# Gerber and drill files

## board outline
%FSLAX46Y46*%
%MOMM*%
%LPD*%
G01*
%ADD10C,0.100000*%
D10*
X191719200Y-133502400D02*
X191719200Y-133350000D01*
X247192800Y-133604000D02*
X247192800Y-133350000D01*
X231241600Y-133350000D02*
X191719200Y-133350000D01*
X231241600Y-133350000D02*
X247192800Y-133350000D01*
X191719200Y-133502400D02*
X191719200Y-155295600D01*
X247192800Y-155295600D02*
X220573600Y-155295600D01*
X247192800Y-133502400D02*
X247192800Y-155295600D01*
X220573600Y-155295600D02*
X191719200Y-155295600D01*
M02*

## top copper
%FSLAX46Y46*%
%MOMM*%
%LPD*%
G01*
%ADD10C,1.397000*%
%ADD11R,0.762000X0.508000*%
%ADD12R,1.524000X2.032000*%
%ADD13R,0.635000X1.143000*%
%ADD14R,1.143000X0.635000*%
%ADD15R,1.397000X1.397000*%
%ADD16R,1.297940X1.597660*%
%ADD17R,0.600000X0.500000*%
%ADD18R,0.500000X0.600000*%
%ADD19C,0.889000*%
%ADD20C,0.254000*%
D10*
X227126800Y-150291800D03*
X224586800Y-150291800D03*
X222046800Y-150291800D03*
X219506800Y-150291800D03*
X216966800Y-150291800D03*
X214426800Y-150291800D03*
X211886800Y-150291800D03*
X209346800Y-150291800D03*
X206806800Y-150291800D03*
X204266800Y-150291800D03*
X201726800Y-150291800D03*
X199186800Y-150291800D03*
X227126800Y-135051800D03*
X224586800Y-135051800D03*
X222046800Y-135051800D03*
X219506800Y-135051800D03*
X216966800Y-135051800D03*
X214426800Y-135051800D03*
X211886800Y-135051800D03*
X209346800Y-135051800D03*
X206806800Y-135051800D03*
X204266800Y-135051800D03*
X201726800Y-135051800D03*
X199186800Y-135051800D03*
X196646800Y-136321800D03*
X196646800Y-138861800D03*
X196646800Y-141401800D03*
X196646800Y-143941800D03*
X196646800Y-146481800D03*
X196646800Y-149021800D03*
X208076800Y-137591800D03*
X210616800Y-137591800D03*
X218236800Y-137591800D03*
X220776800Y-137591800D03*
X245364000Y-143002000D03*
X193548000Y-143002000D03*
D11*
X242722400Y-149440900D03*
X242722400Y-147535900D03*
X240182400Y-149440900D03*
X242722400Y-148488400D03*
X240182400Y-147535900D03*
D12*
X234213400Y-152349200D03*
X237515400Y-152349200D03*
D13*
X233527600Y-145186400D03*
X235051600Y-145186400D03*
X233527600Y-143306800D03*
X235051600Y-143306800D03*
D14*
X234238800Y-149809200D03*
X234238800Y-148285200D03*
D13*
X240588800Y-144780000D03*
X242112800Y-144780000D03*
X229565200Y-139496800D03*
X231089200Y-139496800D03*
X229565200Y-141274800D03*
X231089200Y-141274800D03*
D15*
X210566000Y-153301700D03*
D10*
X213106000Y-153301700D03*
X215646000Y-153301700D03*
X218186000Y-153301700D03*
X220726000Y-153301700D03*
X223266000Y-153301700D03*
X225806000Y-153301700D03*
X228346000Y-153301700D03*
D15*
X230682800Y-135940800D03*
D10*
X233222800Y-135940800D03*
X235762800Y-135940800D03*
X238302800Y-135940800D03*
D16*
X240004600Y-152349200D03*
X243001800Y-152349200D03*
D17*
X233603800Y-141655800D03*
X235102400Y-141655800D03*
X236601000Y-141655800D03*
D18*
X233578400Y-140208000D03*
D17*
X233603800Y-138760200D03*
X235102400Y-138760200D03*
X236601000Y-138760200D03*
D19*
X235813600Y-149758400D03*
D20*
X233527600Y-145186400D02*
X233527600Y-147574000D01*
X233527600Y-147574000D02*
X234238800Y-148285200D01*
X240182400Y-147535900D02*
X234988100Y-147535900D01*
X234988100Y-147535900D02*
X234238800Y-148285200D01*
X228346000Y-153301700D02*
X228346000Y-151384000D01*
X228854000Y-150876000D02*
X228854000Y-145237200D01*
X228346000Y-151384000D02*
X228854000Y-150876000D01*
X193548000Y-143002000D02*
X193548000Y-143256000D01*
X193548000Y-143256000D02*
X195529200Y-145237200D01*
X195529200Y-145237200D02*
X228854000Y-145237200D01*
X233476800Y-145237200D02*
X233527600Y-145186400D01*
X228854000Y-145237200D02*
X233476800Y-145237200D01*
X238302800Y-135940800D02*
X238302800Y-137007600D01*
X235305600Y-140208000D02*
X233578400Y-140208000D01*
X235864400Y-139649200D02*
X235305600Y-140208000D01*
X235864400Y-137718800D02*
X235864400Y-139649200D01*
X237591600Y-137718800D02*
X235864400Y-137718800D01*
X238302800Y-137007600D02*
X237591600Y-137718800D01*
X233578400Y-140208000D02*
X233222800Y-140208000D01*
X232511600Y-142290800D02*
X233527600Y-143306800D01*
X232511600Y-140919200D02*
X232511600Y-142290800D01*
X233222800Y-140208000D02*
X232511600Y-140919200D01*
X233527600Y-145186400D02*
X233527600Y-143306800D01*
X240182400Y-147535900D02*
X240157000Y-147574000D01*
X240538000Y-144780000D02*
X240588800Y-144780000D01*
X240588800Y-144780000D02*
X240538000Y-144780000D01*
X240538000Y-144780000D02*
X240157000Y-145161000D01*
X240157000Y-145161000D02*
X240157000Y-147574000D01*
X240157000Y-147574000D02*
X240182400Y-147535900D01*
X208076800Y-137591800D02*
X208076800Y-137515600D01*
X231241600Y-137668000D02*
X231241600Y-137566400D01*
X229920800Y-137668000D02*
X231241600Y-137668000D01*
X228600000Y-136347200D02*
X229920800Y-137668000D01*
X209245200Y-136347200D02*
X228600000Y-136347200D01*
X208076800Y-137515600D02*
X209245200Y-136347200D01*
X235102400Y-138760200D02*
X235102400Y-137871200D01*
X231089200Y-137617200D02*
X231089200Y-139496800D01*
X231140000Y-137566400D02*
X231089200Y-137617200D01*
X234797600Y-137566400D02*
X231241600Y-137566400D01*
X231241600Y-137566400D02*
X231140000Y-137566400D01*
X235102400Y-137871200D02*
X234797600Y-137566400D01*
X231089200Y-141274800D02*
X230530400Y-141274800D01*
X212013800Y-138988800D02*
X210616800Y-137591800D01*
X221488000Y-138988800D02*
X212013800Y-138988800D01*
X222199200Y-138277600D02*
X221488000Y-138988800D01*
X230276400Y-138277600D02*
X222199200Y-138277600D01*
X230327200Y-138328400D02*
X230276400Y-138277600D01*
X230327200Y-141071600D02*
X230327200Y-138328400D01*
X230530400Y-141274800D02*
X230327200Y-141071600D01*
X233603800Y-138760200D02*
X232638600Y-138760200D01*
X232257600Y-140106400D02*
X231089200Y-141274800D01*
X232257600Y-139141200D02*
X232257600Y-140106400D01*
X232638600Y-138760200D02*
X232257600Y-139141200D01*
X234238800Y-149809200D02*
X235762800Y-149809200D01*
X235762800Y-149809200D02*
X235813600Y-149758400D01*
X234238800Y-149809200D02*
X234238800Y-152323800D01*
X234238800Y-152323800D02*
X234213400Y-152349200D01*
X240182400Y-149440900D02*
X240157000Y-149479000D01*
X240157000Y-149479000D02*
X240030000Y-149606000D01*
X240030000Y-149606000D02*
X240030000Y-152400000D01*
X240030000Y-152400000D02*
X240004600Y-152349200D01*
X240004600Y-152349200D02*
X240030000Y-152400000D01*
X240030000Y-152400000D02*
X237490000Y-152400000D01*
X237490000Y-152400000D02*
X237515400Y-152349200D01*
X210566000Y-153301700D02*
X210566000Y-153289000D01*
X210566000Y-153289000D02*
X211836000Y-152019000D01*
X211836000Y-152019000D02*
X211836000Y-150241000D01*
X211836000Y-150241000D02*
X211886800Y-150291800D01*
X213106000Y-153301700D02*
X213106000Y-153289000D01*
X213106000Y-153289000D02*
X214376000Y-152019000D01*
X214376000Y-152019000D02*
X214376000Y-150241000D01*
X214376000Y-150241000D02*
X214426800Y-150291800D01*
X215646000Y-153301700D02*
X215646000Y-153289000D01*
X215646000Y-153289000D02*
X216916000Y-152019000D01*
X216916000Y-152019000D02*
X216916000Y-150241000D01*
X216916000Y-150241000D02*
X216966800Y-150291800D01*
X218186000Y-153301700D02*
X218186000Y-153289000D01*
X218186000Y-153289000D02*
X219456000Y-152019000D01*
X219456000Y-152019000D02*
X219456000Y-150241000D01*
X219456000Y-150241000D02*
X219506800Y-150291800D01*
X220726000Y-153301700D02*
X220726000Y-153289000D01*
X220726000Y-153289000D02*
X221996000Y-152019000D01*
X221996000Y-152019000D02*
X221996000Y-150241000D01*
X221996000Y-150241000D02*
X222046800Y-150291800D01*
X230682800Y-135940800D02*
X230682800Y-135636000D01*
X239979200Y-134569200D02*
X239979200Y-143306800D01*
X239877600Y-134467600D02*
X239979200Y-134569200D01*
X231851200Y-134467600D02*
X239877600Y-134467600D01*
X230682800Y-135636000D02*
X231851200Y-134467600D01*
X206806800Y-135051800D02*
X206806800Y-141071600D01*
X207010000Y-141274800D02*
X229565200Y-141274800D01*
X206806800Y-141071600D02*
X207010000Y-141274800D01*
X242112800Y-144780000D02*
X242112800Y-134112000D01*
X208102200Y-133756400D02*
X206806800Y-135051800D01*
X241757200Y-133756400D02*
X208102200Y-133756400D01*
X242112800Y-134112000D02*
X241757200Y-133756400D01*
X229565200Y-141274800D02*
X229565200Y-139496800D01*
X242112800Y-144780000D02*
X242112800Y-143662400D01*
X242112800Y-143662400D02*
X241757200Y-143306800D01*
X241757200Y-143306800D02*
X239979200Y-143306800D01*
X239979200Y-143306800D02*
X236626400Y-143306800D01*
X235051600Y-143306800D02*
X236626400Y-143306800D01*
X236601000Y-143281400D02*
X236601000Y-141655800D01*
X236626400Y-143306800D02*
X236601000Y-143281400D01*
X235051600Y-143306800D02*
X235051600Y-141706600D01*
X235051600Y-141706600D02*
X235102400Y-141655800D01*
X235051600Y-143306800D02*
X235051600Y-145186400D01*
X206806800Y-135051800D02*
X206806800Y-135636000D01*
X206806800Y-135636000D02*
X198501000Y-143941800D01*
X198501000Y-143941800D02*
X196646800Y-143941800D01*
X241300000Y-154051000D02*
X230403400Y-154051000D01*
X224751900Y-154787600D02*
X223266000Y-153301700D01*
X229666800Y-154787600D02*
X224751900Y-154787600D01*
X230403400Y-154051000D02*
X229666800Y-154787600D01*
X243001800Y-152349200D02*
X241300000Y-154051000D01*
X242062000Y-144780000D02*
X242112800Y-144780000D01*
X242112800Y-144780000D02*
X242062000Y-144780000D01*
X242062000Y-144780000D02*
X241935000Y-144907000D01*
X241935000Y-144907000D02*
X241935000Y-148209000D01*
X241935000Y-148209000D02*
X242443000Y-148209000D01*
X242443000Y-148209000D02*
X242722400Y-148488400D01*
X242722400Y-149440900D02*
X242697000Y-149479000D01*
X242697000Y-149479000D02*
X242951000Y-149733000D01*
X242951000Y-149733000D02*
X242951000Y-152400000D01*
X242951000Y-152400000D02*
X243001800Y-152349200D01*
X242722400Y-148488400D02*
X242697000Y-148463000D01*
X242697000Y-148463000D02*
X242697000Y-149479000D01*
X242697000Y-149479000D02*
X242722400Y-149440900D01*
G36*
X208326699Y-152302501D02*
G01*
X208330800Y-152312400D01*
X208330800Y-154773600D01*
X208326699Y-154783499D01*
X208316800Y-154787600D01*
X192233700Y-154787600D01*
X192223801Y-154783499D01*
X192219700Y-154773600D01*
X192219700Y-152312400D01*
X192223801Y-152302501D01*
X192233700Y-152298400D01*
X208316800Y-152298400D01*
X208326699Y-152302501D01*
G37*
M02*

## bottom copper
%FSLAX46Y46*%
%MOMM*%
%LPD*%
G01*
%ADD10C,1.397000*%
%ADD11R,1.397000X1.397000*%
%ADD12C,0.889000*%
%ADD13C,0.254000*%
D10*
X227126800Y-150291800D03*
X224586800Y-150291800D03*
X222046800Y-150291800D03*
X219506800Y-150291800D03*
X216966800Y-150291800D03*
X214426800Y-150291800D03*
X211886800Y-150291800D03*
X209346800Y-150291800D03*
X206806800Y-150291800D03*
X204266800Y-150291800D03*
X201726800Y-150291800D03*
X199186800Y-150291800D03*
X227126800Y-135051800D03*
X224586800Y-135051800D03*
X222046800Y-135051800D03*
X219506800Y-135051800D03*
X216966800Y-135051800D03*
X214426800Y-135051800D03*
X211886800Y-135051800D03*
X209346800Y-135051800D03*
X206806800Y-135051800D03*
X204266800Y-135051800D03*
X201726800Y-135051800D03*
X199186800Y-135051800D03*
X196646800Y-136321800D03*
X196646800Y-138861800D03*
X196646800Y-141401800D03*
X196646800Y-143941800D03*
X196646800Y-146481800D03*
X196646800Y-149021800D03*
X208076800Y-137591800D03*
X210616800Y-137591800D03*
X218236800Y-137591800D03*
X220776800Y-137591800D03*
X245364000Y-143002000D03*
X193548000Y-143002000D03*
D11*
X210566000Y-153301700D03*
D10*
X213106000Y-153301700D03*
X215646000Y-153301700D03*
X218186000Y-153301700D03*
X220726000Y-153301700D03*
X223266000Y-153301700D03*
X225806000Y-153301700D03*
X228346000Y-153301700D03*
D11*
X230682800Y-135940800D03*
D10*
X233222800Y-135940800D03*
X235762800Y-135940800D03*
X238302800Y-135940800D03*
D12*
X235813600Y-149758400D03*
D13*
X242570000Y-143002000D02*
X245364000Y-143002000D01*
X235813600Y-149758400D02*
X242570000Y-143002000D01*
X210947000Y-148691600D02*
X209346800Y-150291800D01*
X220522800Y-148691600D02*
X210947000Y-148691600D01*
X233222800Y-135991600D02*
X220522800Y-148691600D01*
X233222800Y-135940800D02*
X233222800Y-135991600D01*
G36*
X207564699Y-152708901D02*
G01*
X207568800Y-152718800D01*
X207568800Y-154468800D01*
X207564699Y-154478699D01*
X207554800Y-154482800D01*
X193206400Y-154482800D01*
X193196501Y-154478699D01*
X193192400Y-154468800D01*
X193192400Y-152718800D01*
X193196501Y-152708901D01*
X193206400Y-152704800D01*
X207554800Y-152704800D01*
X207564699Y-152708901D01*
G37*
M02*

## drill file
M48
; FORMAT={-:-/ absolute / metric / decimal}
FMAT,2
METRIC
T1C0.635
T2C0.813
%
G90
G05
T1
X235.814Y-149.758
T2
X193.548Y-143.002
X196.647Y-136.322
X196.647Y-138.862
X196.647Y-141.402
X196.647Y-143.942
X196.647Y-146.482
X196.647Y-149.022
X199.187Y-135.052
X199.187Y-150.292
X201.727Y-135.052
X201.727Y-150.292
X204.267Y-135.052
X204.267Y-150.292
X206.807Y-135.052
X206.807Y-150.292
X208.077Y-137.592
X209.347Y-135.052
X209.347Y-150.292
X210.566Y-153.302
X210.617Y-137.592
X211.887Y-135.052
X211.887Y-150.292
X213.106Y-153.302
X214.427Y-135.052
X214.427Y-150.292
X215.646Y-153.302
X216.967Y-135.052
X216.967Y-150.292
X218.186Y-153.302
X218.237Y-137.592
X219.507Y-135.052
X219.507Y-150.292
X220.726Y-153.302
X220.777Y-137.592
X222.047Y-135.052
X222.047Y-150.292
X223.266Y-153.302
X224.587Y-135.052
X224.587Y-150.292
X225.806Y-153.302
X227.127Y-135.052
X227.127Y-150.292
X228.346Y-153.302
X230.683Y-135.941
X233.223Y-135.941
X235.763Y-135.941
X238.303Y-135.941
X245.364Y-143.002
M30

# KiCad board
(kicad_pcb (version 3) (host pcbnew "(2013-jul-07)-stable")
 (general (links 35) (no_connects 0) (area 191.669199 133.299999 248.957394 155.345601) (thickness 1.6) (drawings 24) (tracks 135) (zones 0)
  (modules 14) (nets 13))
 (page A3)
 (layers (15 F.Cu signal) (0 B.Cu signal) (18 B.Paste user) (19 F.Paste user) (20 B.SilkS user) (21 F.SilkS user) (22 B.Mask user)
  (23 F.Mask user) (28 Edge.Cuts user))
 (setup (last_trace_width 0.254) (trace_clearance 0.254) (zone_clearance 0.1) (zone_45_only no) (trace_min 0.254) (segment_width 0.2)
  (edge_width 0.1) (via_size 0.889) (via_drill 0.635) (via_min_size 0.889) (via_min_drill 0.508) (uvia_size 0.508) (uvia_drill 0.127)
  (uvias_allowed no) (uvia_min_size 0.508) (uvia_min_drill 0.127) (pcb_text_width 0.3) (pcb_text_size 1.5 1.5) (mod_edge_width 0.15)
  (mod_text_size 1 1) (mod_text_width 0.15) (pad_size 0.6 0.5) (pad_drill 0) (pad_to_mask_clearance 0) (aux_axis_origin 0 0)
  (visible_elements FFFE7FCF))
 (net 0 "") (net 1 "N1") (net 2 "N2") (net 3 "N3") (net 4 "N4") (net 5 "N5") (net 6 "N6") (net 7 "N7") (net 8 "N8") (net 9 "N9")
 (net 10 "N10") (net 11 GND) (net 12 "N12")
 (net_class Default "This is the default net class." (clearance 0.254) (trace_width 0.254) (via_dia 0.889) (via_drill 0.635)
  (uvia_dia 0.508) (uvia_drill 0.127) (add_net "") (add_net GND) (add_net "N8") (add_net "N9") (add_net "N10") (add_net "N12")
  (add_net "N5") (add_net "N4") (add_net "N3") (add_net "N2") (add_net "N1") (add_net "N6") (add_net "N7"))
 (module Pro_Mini (layer F.Cu) (at 211.9884 142.6972)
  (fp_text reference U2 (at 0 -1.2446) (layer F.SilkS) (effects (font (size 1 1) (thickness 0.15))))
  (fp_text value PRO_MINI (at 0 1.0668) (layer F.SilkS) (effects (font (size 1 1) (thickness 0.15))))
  (pad 9 thru_hole circle (at 15.1384 7.5946) (size 1.397 1.397) (drill 0.8128) (layers *.Cu *.Mask F.SilkS))
  (pad 8 thru_hole circle (at 12.5984 7.5946) (size 1.397 1.397) (drill 0.8128) (layers *.Cu *.Mask F.SilkS))
  (pad 7 thru_hole circle (at 10.0584 7.5946) (size 1.397 1.397) (drill 0.8128) (layers *.Cu *.Mask F.SilkS) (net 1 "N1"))
  (pad 6 thru_hole circle (at 7.5184 7.5946) (size 1.397 1.397) (drill 0.8128) (layers *.Cu *.Mask F.SilkS) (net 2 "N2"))
  (pad 5 thru_hole circle (at 4.9784 7.5946) (size 1.397 1.397) (drill 0.8128) (layers *.Cu *.Mask F.SilkS) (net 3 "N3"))
  (pad 4 thru_hole circle (at 2.4384 7.5946) (size 1.397 1.397) (drill 0.8128) (layers *.Cu *.Mask F.SilkS) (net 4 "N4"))
  (pad 3 thru_hole circle (at -0.1016 7.5946) (size 1.397 1.397) (drill 0.8128) (layers *.Cu *.Mask F.SilkS) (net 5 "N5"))
  (pad 2 thru_hole circle (at -2.6416 7.5946) (size 1.397 1.397) (drill 0.8128) (layers *.Cu *.Mask F.SilkS) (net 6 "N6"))
  (pad GND thru_hole circle (at -5.1816 7.5946) (size 1.397 1.397) (drill 0.8128) (layers *.Cu *.Mask F.SilkS))
  (pad RST thru_hole circle (at -7.7216 7.5946) (size 1.397 1.397) (drill 0.8128) (layers *.Cu *.Mask F.SilkS))
  (pad RX1 thru_hole circle (at -10.2616 7.5946) (size 1.397 1.397) (drill 0.8128) (layers *.Cu *.Mask F.SilkS))
  (pad TX0 thru_hole circle (at -12.8016 7.5946) (size 1.397 1.397) (drill 0.8128) (layers *.Cu *.Mask F.SilkS))
  (pad 10 thru_hole circle (at 15.1384 -7.6454) (size 1.397 1.397) (drill 0.8128) (layers *.Cu *.Mask F.SilkS))
  (pad 11 thru_hole circle (at 12.5984 -7.6454) (size 1.397 1.397) (drill 0.8128) (layers *.Cu *.Mask F.SilkS))
  (pad 12 thru_hole circle (at 10.0584 -7.6454) (size 1.397 1.397) (drill 0.8128) (layers *.Cu *.Mask F.SilkS))
  (pad 13 thru_hole circle (at 7.5184 -7.6454) (size 1.397 1.397) (drill 0.8128) (layers *.Cu *.Mask F.SilkS))
  (pad A0 thru_hole circle (at 4.9784 -7.6454) (size 1.397 1.397) (drill 0.8128) (layers *.Cu *.Mask F.SilkS))
  (pad A1 thru_hole circle (at 2.4384 -7.6454) (size 1.397 1.397) (drill 0.8128) (layers *.Cu *.Mask F.SilkS))
  (pad A2 thru_hole circle (at -0.1016 -7.6454) (size 1.397 1.397) (drill 0.8128) (layers *.Cu *.Mask F.SilkS))
  (pad A3 thru_hole circle (at -2.6416 -7.6454) (size 1.397 1.397) (drill 0.8128) (layers *.Cu *.Mask F.SilkS))
  (pad VCC thru_hole circle (at -5.1816 -7.6454) (size 1.397 1.397) (drill 0.8128) (layers *.Cu *.Mask F.SilkS) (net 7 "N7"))
  (pad RST thru_hole circle (at -7.7216 -7.6454) (size 1.397 1.397) (drill 0.8128) (layers *.Cu *.Mask F.SilkS))
  (pad GND thru_hole circle (at -10.2616 -7.6454) (size 1.397 1.397) (drill 0.8128) (layers *.Cu *.Mask F.SilkS))
  (pad RAW thru_hole circle (at -12.8016 -7.6454) (size 1.397 1.397) (drill 0.8128) (layers *.Cu *.Mask F.SilkS))
  (pad GRN thru_hole circle (at -15.3416 -6.3754) (size 1.397 1.397) (drill 0.8128) (layers *.Cu *.Mask F.SilkS))
  (pad TX0 thru_hole circle (at -15.3416 -3.8354) (size 1.397 1.397) (drill 0.8128) (layers *.Cu *.Mask F.SilkS))
  (pad RX1 thru_hole circle (at -15.3416 -1.2954) (size 1.397 1.397) (drill 0.8128) (layers *.Cu *.Mask F.SilkS))
  (pad VCC thru_hole circle (at -15.3416 1.2446) (size 1.397 1.397) (drill 0.8128) (layers *.Cu *.Mask F.SilkS) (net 7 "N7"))
  (pad GND thru_hole circle (at -15.3416 3.7846) (size 1.397 1.397) (drill 0.8128) (layers *.Cu *.Mask F.SilkS))
  (pad BLK thru_hole circle (at -15.3416 6.3246) (size 1.397 1.397) (drill 0.8128) (layers *.Cu *.Mask F.SilkS))
  (pad A5 thru_hole circle (at -3.9116 -5.1054) (size 1.397 1.397) (drill 0.8128) (layers *.Cu *.Mask F.SilkS) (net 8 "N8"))
  (pad A4 thru_hole circle (at -1.3716 -5.1054) (size 1.397 1.397) (drill 0.8128) (layers *.Cu *.Mask F.SilkS) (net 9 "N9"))
  (pad A7 thru_hole circle (at 6.2484 -5.1054) (size 1.397 1.397) (drill 0.8128) (layers *.Cu *.Mask F.SilkS))
  (pad A6 thru_hole circle (at 8.7884 -5.1054) (size 1.397 1.397) (drill 0.8128) (layers *.Cu *.Mask F.SilkS)))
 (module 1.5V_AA (layer B.Cu) (at 219.456 143.002)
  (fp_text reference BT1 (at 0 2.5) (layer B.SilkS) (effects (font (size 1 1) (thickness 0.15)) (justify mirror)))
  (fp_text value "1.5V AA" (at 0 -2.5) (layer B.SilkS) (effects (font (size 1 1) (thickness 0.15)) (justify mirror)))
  (pad 1 thru_hole circle (at 25.908 0) (size 1.397 1.397) (drill 0.8128) (layers *.Cu *.Mask B.SilkS) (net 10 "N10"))
  (pad 2 thru_hole circle (at -25.908 0) (size 1.397 1.397) (drill 0.8128) (layers *.Cu *.Mask B.SilkS) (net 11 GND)))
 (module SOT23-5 (layer F.Cu) (at 241.4524 148.4884 90)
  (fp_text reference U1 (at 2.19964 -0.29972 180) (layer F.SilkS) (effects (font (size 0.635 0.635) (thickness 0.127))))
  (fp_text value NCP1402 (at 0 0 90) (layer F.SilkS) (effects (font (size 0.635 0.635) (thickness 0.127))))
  (pad 1 smd rect (at -0.9525 1.27 90) (size 0.508 0.762) (layers F.Cu F.Paste F.Mask) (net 7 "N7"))
  (pad 3 smd rect (at 0.9525 1.27 90) (size 0.508 0.762) (layers F.Cu F.Paste F.Mask))
  (pad 5 smd rect (at -0.9525 -1.27 90) (size 0.508 0.762) (layers F.Cu F.Paste F.Mask) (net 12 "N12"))
  (pad 2 smd rect (at 0 1.27 90) (size 0.508 0.762) (layers F.Cu F.Paste F.Mask) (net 7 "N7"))
  (pad 4 smd rect (at 0.9525 -1.27 90) (size 0.508 0.762) (layers F.Cu F.Paste F.Mask) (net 11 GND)))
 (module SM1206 (layer F.Cu) (at 235.8644 152.3492)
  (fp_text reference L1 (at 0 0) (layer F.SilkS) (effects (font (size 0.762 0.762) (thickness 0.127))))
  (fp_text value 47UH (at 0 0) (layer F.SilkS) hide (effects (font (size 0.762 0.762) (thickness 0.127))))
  (pad 1 smd rect (at -1.651 0) (size 1.524 2.032) (layers F.Cu F.Paste F.Mask) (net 10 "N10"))
  (pad 2 smd rect (at 1.651 0) (size 1.524 2.032) (layers F.Cu F.Paste F.Mask) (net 12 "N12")))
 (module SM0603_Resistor (layer F.Cu) (at 234.2896 145.1864)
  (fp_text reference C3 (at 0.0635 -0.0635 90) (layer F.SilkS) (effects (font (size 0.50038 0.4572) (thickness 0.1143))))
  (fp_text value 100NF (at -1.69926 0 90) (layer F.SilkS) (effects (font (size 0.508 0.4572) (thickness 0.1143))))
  (pad 1 smd rect (at -0.762 0) (size 0.635 1.143) (layers F.Cu F.Paste F.Mask) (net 11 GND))
  (pad 2 smd rect (at 0.762 0) (size 0.635 1.143) (layers F.Cu F.Paste F.Mask) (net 7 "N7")))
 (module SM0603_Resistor (layer F.Cu) (at 234.2896 143.3068)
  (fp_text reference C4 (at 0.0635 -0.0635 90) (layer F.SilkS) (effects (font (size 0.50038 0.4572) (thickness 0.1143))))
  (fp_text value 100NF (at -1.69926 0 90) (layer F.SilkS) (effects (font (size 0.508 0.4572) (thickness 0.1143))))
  (pad 1 smd rect (at -0.762 0) (size 0.635 1.143) (layers F.Cu F.Paste F.Mask) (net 11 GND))
  (pad 2 smd rect (at 0.762 0) (size 0.635 1.143) (layers F.Cu F.Paste F.Mask) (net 7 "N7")))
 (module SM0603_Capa (layer F.Cu) (at 234.2388 149.0472 90)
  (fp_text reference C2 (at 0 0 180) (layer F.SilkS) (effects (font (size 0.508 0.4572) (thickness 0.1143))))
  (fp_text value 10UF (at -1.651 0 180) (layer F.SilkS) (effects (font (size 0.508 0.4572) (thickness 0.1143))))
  (pad 1 smd rect (at -0.762 0 90) (size 0.635 1.143) (layers F.Cu F.Paste F.Mask) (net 10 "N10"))
  (pad 2 smd rect (at 0.762 0 90) (size 0.635 1.143) (layers F.Cu F.Paste F.Mask) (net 11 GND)))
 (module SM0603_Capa (layer F.Cu) (at 241.3508 144.78)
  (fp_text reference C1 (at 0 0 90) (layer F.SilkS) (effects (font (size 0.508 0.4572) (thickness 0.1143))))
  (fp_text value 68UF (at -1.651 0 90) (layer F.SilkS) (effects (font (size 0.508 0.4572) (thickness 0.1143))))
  (pad 1 smd rect (at -0.762 0) (size 0.635 1.143) (layers F.Cu F.Paste F.Mask) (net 11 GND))
  (pad 2 smd rect (at 0.762 0) (size 0.635 1.143) (layers F.Cu F.Paste F.Mask) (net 7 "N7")))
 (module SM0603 (layer F.Cu) (at 230.3272 139.4968)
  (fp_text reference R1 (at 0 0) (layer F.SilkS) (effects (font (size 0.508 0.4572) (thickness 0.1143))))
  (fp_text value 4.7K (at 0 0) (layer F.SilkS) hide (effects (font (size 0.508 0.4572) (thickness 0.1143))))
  (pad 1 smd rect (at -0.762 0) (size 0.635 1.143) (layers F.Cu F.Paste F.Mask) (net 7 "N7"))
  (pad 2 smd rect (at 0.762 0) (size 0.635 1.143) (layers F.Cu F.Paste F.Mask) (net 8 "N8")))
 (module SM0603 (layer F.Cu) (at 230.3272 141.2748)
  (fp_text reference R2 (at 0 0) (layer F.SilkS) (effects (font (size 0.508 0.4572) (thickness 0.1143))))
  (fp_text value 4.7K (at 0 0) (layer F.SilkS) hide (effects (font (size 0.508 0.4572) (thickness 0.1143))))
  (pad 1 smd rect (at -0.762 0) (size 0.635 1.143) (layers F.Cu F.Paste F.Mask) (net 7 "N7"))
  (pad 2 smd rect (at 0.762 0) (size 0.635 1.143) (layers F.Cu F.Paste F.Mask) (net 9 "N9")))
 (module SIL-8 (layer F.Cu) (at 219.456 153.3017)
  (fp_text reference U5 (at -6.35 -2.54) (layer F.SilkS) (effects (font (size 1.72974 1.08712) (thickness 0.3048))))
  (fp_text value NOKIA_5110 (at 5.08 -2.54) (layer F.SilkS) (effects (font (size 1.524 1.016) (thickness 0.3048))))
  (pad 1 thru_hole rect (at -8.89 0) (size 1.397 1.397) (drill 0.8128) (layers *.Cu *.Mask F.SilkS) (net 5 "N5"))
  (pad 2 thru_hole circle (at -6.35 0) (size 1.397 1.397) (drill 0.8128) (layers *.Cu *.Mask F.SilkS) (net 4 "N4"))
  (pad 3 thru_hole circle (at -3.81 0) (size 1.397 1.397) (drill 0.8128) (layers *.Cu *.Mask F.SilkS) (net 3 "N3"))
  (pad 4 thru_hole circle (at -1.27 0) (size 1.397 1.397) (drill 0.8128) (layers *.Cu *.Mask F.SilkS) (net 2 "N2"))
  (pad 5 thru_hole circle (at 1.27 0) (size 1.397 1.397) (drill 0.8128) (layers *.Cu *.Mask F.SilkS) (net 1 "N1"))
  (pad 6 thru_hole circle (at 3.81 0) (size 1.397 1.397) (drill 0.8128) (layers *.Cu *.Mask F.SilkS) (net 7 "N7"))
  (pad 7 thru_hole circle (at 6.35 0) (size 1.397 1.397) (drill 0.8128) (layers *.Cu *.Mask F.SilkS))
  (pad 8 thru_hole circle (at 8.89 0) (size 1.397 1.397) (drill 0.8128) (layers *.Cu *.Mask F.SilkS) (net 11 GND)))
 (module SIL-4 (layer B.Cu) (at 234.4928 135.9408)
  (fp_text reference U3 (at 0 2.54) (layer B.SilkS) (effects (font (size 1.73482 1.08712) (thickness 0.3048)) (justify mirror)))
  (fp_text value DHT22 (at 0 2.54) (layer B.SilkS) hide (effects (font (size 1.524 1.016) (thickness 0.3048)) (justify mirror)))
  (pad 1 thru_hole rect (at -3.81 0) (size 1.397 1.397) (drill 0.8128) (layers *.Cu *.Mask B.SilkS) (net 7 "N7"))
  (pad 2 thru_hole circle (at -1.27 0) (size 1.397 1.397) (drill 0.8128) (layers *.Cu *.Mask B.SilkS) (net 6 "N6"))
  (pad 3 thru_hole circle (at 1.27 0) (size 1.397 1.397) (drill 0.8128) (layers *.Cu *.Mask B.SilkS))
  (pad 4 thru_hole circle (at 3.81 0) (size 1.397 1.397) (drill 0.8128) (layers *.Cu *.Mask B.SilkS) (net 11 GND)))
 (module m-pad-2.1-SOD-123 (layer F.Cu) (at 241.5032 152.3492)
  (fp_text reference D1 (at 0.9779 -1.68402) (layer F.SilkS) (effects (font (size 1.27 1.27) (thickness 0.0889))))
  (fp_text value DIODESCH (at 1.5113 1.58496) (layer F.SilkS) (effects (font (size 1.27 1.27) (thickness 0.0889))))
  (pad 1 smd rect (at -1.4986 0) (size 1.29794 1.59766) (layers F.Cu F.Paste F.Mask) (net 12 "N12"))
  (pad 2 smd rect (at 1.4986 0) (size 1.29794 1.59766) (layers F.Cu F.Paste F.Mask) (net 7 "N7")))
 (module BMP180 (layer F.Cu) (at 235.1024 140.208 180)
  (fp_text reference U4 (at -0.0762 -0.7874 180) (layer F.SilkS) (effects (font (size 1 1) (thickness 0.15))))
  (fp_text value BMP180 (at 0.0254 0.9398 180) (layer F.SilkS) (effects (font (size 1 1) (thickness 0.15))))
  (pad 1 smd rect (at 1.4986 -1.4478 180) (size 0.6 0.5) (layers F.Cu F.Paste F.Mask))
  (pad 2 smd rect (at 0 -1.4478 180) (size 0.6 0.5) (layers F.Cu F.Paste F.Mask) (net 7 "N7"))
  (pad 3 smd rect (at -1.4986 -1.4478 180) (size 0.6 0.5) (layers F.Cu F.Paste F.Mask) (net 7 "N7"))
  (pad 7 smd rect (at 1.524 0 180) (size 0.5 0.6) (layers F.Cu F.Paste F.Mask) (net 11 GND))
  (pad 6 smd rect (at 1.4986 1.4478 180) (size 0.6 0.5) (layers F.Cu F.Paste F.Mask) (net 9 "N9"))
  (pad 5 smd rect (at 0 1.4478 180) (size 0.6 0.5) (layers F.Cu F.Paste F.Mask) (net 8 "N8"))
  (pad 4 smd rect (at -1.4986 1.4478 180) (size 0.6 0.5) (layers F.Cu F.Paste F.Mask)))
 (gr_line (start 191.7192 133.5024) (end 191.7192 133.35) (angle 90) (layer Edge.Cuts) (width 0.1))
 (gr_line (start 247.1928 133.604) (end 247.1928 133.35) (angle 90) (layer Edge.Cuts) (width 0.1))
 (gr_line (start 231.2416 133.35) (end 191.7192 133.35) (angle 90) (layer Edge.Cuts) (width 0.1))
 (gr_line (start 231.2416 133.35) (end 247.1928 133.35) (angle 90) (layer Edge.Cuts) (width 0.1))
 (gr_line (start 191.7192 133.5024) (end 191.7192 155.2956) (angle 90) (layer Edge.Cuts) (width 0.1))
 (gr_line (start 247.1928 155.2956) (end 220.5736 155.2956) (angle 90) (layer Edge.Cuts) (width 0.1))
 (gr_line (start 247.1928 133.5024) (end 247.1928 155.2956) (angle 90) (layer Edge.Cuts) (width 0.1))
 (gr_line (start 220.5736 155.2956) (end 191.7192 155.2956) (angle 90) (layer Edge.Cuts) (width 0.1))
 (segment (start 233.5276 145.1864) (end 233.5276 147.574) (width 0.254) (layer F.Cu) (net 11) (status 400000))
 (segment (start 233.5276 147.574) (end 234.2388 148.2852) (width 0.254) (layer F.Cu) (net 11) (status 800000))
 (segment (start 240.1824 147.5359) (end 234.9881 147.5359) (width 0.254) (layer F.Cu) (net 11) (status 400000))
 (segment (start 234.9881 147.5359) (end 234.2388 148.2852) (width 0.254) (layer F.Cu) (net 11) (status 800000))
 (segment (start 228.346 153.3017) (end 228.346 151.384) (width 0.254) (layer F.Cu) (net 11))
 (segment (start 228.854 150.876) (end 228.854 145.2372) (width 0.254) (layer F.Cu) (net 11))
 (segment (start 228.346 151.384) (end 228.854 150.876) (width 0.254) (layer F.Cu) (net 11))
 (segment (start 193.548 143.002) (end 193.548 143.256) (width 0.254) (layer F.Cu) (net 11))
 (segment (start 193.548 143.256) (end 195.5292 145.2372) (width 0.254) (layer F.Cu) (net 11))
 (segment (start 195.5292 145.2372) (end 228.854 145.2372) (width 0.254) (layer F.Cu) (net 11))
 (segment (start 233.4768 145.2372) (end 233.5276 145.1864) (width 0.254) (layer F.Cu) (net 11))
 (segment (start 228.854 145.2372) (end 233.4768 145.2372) (width 0.254) (layer F.Cu) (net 11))
 (segment (start 238.3028 135.9408) (end 238.3028 137.0076) (width 0.254) (layer F.Cu) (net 11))
 (segment (start 235.3056 140.208) (end 233.5784 140.208) (width 0.254) (layer F.Cu) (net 11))
 (segment (start 235.8644 139.6492) (end 235.3056 140.208) (width 0.254) (layer F.Cu) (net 11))
 (segment (start 235.8644 137.7188) (end 235.8644 139.6492) (width 0.254) (layer F.Cu) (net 11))
 (segment (start 237.5916 137.7188) (end 235.8644 137.7188) (width 0.254) (layer F.Cu) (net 11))
 (segment (start 238.3028 137.0076) (end 237.5916 137.7188) (width 0.254) (layer F.Cu) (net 11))
 (segment (start 233.5784 140.208) (end 233.2228 140.208) (width 0.254) (layer F.Cu) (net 11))
 (segment (start 232.5116 142.2908) (end 233.5276 143.3068) (width 0.254) (layer F.Cu) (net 11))
 (segment (start 232.5116 140.9192) (end 232.5116 142.2908) (width 0.254) (layer F.Cu) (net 11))
 (segment (start 233.2228 140.208) (end 232.5116 140.9192) (width 0.254) (layer F.Cu) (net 11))
 (segment (start 233.5276 145.1864) (end 233.5276 143.3068) (width 0.254) (layer F.Cu) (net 11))
 (segment (start 240.1824 147.5359) (end 240.157 147.574) (width 0.254) (layer F.Cu) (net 11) (status 80000))
 (segment (start 240.538 144.78) (end 240.5888 144.78) (width 0.254) (layer F.Cu) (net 11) (status 80000))
 (segment (start 240.5888 144.78) (end 240.538 144.78) (width 0.254) (layer F.Cu) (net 11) (status 80000))
 (segment (start 240.538 144.78) (end 240.157 145.161) (width 0.254) (layer F.Cu) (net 11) (status 80000))
 (segment (start 240.157 145.161) (end 240.157 147.574) (width 0.254) (layer F.Cu) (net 11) (status 80000))
 (segment (start 240.157 147.574) (end 240.1824 147.5359) (width 0.254) (layer F.Cu) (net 11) (status 80000))
 (segment (start 208.0768 137.5918) (end 208.0768 137.5156) (width 0.254) (layer F.Cu) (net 8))
 (segment (start 231.2416 137.668) (end 231.2416 137.5664) (width 0.254) (layer F.Cu) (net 8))
 (segment (start 229.9208 137.668) (end 231.2416 137.668) (width 0.254) (layer F.Cu) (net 8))
 (segment (start 228.6 136.3472) (end 229.9208 137.668) (width 0.254) (layer F.Cu) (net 8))
 (segment (start 209.2452 136.3472) (end 228.6 136.3472) (width 0.254) (layer F.Cu) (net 8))
 (segment (start 208.0768 137.5156) (end 209.2452 136.3472) (width 0.254) (layer F.Cu) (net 8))
 (segment (start 235.1024 138.7602) (end 235.1024 137.8712) (width 0.254) (layer F.Cu) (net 8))
 (segment (start 231.0892 137.6172) (end 231.0892 139.4968) (width 0.254) (layer F.Cu) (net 8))
 (segment (start 231.14 137.5664) (end 231.0892 137.6172) (width 0.254) (layer F.Cu) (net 8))
 (segment (start 234.7976 137.5664) (end 231.2416 137.5664) (width 0.254) (layer F.Cu) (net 8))
 (segment (start 231.2416 137.5664) (end 231.14 137.5664) (width 0.254) (layer F.Cu) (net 8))
 (segment (start 235.1024 137.8712) (end 234.7976 137.5664) (width 0.254) (layer F.Cu) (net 8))
 (segment (start 231.0892 141.2748) (end 230.5304 141.2748) (width 0.254) (layer F.Cu) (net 9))
 (segment (start 212.0138 138.9888) (end 210.6168 137.5918) (width 0.254) (layer F.Cu) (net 9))
 (segment (start 221.488 138.9888) (end 212.0138 138.9888) (width 0.254) (layer F.Cu) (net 9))
 (segment (start 222.1992 138.2776) (end 221.488 138.9888) (width 0.254) (layer F.Cu) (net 9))
 (segment (start 230.2764 138.2776) (end 222.1992 138.2776) (width 0.254) (layer F.Cu) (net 9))
 (segment (start 230.3272 138.3284) (end 230.2764 138.2776) (width 0.254) (layer F.Cu) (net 9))
 (segment (start 230.3272 141.0716) (end 230.3272 138.3284) (width 0.254) (layer F.Cu) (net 9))
 (segment (start 230.5304 141.2748) (end 230.3272 141.0716) (width 0.254) (layer F.Cu) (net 9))
 (segment (start 233.6038 138.7602) (end 232.6386 138.7602) (width 0.254) (layer F.Cu) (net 9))
 (segment (start 232.2576 140.1064) (end 231.0892 141.2748) (width 0.254) (layer F.Cu) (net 9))
 (segment (start 232.2576 139.1412) (end 232.2576 140.1064) (width 0.254) (layer F.Cu) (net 9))
 (segment (start 232.6386 138.7602) (end 232.2576 139.1412) (width 0.254) (layer F.Cu) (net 9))
 (segment (start 234.2388 149.8092) (end 235.7628 149.8092) (width 0.254) (layer F.Cu) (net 10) (status 400000))
 (segment (start 242.57 143.002) (end 245.364 143.002) (width 0.254) (layer B.Cu) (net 10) (status 800000))
 (segment (start 235.8136 149.7584) (end 242.57 143.002) (width 0.254) (layer B.Cu) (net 10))
 (via (at 235.8136 149.7584) (size 0.889) (layers F.Cu B.Cu) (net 10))
 (segment (start 235.7628 149.8092) (end 235.8136 149.7584) (width 0.254) (layer F.Cu) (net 10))
 (segment (start 234.2388 149.8092) (end 234.2388 152.3238) (width 0.254) (layer F.Cu) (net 10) (status C00000))
 (segment (start 234.2388 152.3238) (end 234.2134 152.3492) (width 0.254) (layer F.Cu) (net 10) (status C00000))
 (segment (start 240.1824 149.4409) (end 240.157 149.479) (width 0.254) (layer F.Cu) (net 12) (status 80000))
 (segment (start 240.157 149.479) (end 240.03 149.606) (width 0.254) (layer F.Cu) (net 12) (status 80000))
 (segment (start 240.03 149.606) (end 240.03 152.4) (width 0.254) (layer F.Cu) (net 12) (status 80000))
 (segment (start 240.03 152.4) (end 240.0046 152.3492) (width 0.254) (layer F.Cu) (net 12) (status 80000))
 (segment (start 240.0046 152.3492) (end 240.03 152.4) (width 0.254) (layer F.Cu) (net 12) (status 80000))
 (segment (start 240.03 152.4) (end 237.49 152.4) (width 0.254) (layer F.Cu) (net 12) (status 80000))
 (segment (start 237.49 152.4) (end 237.5154 152.3492) (width 0.254) (layer F.Cu) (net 12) (status 80000))
 (segment (start 210.566 153.3017) (end 210.566 153.289) (width 0.254) (layer F.Cu) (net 5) (status 80000))
 (segment (start 210.566 153.289) (end 211.836 152.019) (width 0.254) (layer F.Cu) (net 5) (status 80000))
 (segment (start 211.836 152.019) (end 211.836 150.241) (width 0.254) (layer F.Cu) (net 5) (status 80000))
 (segment (start 211.836 150.241) (end 211.8868 150.2918) (width 0.254) (layer F.Cu) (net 5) (status 80000))
 (segment (start 213.106 153.3017) (end 213.106 153.289) (width 0.254) (layer F.Cu) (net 4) (status 80000))
 (segment (start 213.106 153.289) (end 214.376 152.019) (width 0.254) (layer F.Cu) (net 4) (status 80000))
 (segment (start 214.376 152.019) (end 214.376 150.241) (width 0.254) (layer F.Cu) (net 4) (status 80000))
 (segment (start 214.376 150.241) (end 214.4268 150.2918) (width 0.254) (layer F.Cu) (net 4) (status 80000))
 (segment (start 215.646 153.3017) (end 215.646 153.289) (width 0.254) (layer F.Cu) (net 3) (status 80000))
 (segment (start 215.646 153.289) (end 216.916 152.019) (width 0.254) (layer F.Cu) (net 3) (status 80000))
 (segment (start 216.916 152.019) (end 216.916 150.241) (width 0.254) (layer F.Cu) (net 3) (status 80000))
 (segment (start 216.916 150.241) (end 216.9668 150.2918) (width 0.254) (layer F.Cu) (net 3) (status 80000))
 (segment (start 218.186 153.3017) (end 218.186 153.289) (width 0.254) (layer F.Cu) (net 2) (status 80000))
 (segment (start 218.186 153.289) (end 219.456 152.019) (width 0.254) (layer F.Cu) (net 2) (status 80000))
 (segment (start 219.456 152.019) (end 219.456 150.241) (width 0.254) (layer F.Cu) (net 2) (status 80000))
 (segment (start 219.456 150.241) (end 219.5068 150.2918) (width 0.254) (layer F.Cu) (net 2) (status 80000))
 (segment (start 220.726 153.3017) (end 220.726 153.289) (width 0.254) (layer F.Cu) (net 1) (status 80000))
 (segment (start 220.726 153.289) (end 221.996 152.019) (width 0.254) (layer F.Cu) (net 1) (status 80000))
 (segment (start 221.996 152.019) (end 221.996 150.241) (width 0.254) (layer F.Cu) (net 1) (status 80000))
 (segment (start 221.996 150.241) (end 222.0468 150.2918) (width 0.254) (layer F.Cu) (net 1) (status 80000))
 (segment (start 210.947 148.6916) (end 209.3468 150.2918) (width 0.254) (layer B.Cu) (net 6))
 (segment (start 220.5228 148.6916) (end 210.947 148.6916) (width 0.254) (layer B.Cu) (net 6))
 (segment (start 233.2228 135.9916) (end 220.5228 148.6916) (width 0.254) (layer B.Cu) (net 6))
 (segment (start 233.2228 135.9408) (end 233.2228 135.9916) (width 0.254) (layer B.Cu) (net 6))
 (segment (start 230.6828 135.9408) (end 230.6828 135.636) (width 0.254) (layer F.Cu) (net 7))
 (segment (start 239.9792 134.5692) (end 239.9792 143.3068) (width 0.254) (layer F.Cu) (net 7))
 (segment (start 239.8776 134.4676) (end 239.9792 134.5692) (width 0.254) (layer F.Cu) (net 7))
 (segment (start 231.8512 134.4676) (end 239.8776 134.4676) (width 0.254) (layer F.Cu) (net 7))
 (segment (start 230.6828 135.636) (end 231.8512 134.4676) (width 0.254) (layer F.Cu) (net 7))
 (segment (start 206.8068 135.0518) (end 206.8068 141.0716) (width 0.254) (layer F.Cu) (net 7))
 (segment (start 207.01 141.2748) (end 229.5652 141.2748) (width 0.254) (layer F.Cu) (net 7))
 (segment (start 206.8068 141.0716) (end 207.01 141.2748) (width 0.254) (layer F.Cu) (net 7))
 (segment (start 242.1128 144.78) (end 242.1128 134.112) (width 0.254) (layer F.Cu) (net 7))
 (segment (start 208.1022 133.7564) (end 206.8068 135.0518) (width 0.254) (layer F.Cu) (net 7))
 (segment (start 241.7572 133.7564) (end 208.1022 133.7564) (width 0.254) (layer F.Cu) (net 7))
 (segment (start 242.1128 134.112) (end 241.7572 133.7564) (width 0.254) (layer F.Cu) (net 7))
 (segment (start 229.5652 141.2748) (end 229.5652 139.4968) (width 0.254) (layer F.Cu) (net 7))
 (segment (start 242.1128 144.78) (end 242.1128 143.6624) (width 0.254) (layer F.Cu) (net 7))
 (segment (start 242.1128 143.6624) (end 241.7572 143.3068) (width 0.254) (layer F.Cu) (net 7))
 (segment (start 241.7572 143.3068) (end 239.9792 143.3068) (width 0.254) (layer F.Cu) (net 7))
 (segment (start 239.9792 143.3068) (end 236.6264 143.3068) (width 0.254) (layer F.Cu) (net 7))
 (segment (start 235.0516 143.3068) (end 236.6264 143.3068) (width 0.254) (layer F.Cu) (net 7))
 (segment (start 236.601 143.2814) (end 236.601 141.6558) (width 0.254) (layer F.Cu) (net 7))
 (segment (start 236.6264 143.3068) (end 236.601 143.2814) (width 0.254) (layer F.Cu) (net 7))
 (segment (start 235.0516 143.3068) (end 235.0516 141.7066) (width 0.254) (layer F.Cu) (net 7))
 (segment (start 235.0516 141.7066) (end 235.1024 141.6558) (width 0.254) (layer F.Cu) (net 7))
 (segment (start 235.0516 143.3068) (end 235.0516 145.1864) (width 0.254) (layer F.Cu) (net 7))
 (segment (start 206.8068 135.0518) (end 206.8068 135.636) (width 0.254) (layer F.Cu) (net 7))
 (segment (start 206.8068 135.636) (end 198.501 143.9418) (width 0.254) (layer F.Cu) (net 7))
 (segment (start 198.501 143.9418) (end 196.6468 143.9418) (width 0.254) (layer F.Cu) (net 7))
 (segment (start 241.3 154.051) (end 230.4034 154.051) (width 0.254) (layer F.Cu) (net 7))
 (segment (start 224.7519 154.7876) (end 223.266 153.3017) (width 0.254) (layer F.Cu) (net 7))
 (segment (start 229.6668 154.7876) (end 224.7519 154.7876) (width 0.254) (layer F.Cu) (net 7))
 (segment (start 230.4034 154.051) (end 229.6668 154.7876) (width 0.254) (layer F.Cu) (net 7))
 (segment (start 243.0018 152.3492) (end 241.3 154.051) (width 0.254) (layer F.Cu) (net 7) (status 80000))
 (segment (start 242.062 144.78) (end 242.1128 144.78) (width 0.254) (layer F.Cu) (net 7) (status 80000))
 (segment (start 242.1128 144.78) (end 242.062 144.78) (width 0.254) (layer F.Cu) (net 7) (status 80000))
 (segment (start 242.062 144.78) (end 241.935 144.907) (width 0.254) (layer F.Cu) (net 7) (status 80000))
 (segment (start 241.935 144.907) (end 241.935 148.209) (width 0.254) (layer F.Cu) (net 7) (status 80000))
 (segment (start 241.935 148.209) (end 242.443 148.209) (width 0.254) (layer F.Cu) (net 7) (status 80000))
 (segment (start 242.443 148.209) (end 242.7224 148.4884) (width 0.254) (layer F.Cu) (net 7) (status 80000))
 (segment (start 242.7224 149.4409) (end 242.697 149.479) (width 0.254) (layer F.Cu) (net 7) (status 80000))
 (segment (start 242.697 149.479) (end 242.951 149.733) (width 0.254) (layer F.Cu) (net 7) (status 80000))
 (segment (start 242.951 149.733) (end 242.951 152.4) (width 0.254) (layer F.Cu) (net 7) (status 80000))
 (segment (start 242.951 152.4) (end 243.0018 152.3492) (width 0.254) (layer F.Cu) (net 7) (status 80000))
 (segment (start 242.7224 148.4884) (end 242.697 148.463) (width 0.254) (layer F.Cu) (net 7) (status 80000))
 (segment (start 242.697 148.463) (end 242.697 149.479) (width 0.254) (layer F.Cu) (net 7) (status 80000))
 (segment (start 242.697 149.479) (end 242.7224 149.4409) (width 0.254) (layer F.Cu) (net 7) (status 80000))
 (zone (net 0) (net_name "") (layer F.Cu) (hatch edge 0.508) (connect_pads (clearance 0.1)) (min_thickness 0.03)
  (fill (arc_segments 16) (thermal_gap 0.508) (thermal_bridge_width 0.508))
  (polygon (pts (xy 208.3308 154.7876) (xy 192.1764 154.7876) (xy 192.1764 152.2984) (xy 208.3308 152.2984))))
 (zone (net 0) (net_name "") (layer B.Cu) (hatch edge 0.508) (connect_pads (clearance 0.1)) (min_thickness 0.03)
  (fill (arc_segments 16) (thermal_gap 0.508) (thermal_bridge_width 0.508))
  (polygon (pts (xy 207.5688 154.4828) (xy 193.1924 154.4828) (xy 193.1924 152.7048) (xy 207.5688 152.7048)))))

